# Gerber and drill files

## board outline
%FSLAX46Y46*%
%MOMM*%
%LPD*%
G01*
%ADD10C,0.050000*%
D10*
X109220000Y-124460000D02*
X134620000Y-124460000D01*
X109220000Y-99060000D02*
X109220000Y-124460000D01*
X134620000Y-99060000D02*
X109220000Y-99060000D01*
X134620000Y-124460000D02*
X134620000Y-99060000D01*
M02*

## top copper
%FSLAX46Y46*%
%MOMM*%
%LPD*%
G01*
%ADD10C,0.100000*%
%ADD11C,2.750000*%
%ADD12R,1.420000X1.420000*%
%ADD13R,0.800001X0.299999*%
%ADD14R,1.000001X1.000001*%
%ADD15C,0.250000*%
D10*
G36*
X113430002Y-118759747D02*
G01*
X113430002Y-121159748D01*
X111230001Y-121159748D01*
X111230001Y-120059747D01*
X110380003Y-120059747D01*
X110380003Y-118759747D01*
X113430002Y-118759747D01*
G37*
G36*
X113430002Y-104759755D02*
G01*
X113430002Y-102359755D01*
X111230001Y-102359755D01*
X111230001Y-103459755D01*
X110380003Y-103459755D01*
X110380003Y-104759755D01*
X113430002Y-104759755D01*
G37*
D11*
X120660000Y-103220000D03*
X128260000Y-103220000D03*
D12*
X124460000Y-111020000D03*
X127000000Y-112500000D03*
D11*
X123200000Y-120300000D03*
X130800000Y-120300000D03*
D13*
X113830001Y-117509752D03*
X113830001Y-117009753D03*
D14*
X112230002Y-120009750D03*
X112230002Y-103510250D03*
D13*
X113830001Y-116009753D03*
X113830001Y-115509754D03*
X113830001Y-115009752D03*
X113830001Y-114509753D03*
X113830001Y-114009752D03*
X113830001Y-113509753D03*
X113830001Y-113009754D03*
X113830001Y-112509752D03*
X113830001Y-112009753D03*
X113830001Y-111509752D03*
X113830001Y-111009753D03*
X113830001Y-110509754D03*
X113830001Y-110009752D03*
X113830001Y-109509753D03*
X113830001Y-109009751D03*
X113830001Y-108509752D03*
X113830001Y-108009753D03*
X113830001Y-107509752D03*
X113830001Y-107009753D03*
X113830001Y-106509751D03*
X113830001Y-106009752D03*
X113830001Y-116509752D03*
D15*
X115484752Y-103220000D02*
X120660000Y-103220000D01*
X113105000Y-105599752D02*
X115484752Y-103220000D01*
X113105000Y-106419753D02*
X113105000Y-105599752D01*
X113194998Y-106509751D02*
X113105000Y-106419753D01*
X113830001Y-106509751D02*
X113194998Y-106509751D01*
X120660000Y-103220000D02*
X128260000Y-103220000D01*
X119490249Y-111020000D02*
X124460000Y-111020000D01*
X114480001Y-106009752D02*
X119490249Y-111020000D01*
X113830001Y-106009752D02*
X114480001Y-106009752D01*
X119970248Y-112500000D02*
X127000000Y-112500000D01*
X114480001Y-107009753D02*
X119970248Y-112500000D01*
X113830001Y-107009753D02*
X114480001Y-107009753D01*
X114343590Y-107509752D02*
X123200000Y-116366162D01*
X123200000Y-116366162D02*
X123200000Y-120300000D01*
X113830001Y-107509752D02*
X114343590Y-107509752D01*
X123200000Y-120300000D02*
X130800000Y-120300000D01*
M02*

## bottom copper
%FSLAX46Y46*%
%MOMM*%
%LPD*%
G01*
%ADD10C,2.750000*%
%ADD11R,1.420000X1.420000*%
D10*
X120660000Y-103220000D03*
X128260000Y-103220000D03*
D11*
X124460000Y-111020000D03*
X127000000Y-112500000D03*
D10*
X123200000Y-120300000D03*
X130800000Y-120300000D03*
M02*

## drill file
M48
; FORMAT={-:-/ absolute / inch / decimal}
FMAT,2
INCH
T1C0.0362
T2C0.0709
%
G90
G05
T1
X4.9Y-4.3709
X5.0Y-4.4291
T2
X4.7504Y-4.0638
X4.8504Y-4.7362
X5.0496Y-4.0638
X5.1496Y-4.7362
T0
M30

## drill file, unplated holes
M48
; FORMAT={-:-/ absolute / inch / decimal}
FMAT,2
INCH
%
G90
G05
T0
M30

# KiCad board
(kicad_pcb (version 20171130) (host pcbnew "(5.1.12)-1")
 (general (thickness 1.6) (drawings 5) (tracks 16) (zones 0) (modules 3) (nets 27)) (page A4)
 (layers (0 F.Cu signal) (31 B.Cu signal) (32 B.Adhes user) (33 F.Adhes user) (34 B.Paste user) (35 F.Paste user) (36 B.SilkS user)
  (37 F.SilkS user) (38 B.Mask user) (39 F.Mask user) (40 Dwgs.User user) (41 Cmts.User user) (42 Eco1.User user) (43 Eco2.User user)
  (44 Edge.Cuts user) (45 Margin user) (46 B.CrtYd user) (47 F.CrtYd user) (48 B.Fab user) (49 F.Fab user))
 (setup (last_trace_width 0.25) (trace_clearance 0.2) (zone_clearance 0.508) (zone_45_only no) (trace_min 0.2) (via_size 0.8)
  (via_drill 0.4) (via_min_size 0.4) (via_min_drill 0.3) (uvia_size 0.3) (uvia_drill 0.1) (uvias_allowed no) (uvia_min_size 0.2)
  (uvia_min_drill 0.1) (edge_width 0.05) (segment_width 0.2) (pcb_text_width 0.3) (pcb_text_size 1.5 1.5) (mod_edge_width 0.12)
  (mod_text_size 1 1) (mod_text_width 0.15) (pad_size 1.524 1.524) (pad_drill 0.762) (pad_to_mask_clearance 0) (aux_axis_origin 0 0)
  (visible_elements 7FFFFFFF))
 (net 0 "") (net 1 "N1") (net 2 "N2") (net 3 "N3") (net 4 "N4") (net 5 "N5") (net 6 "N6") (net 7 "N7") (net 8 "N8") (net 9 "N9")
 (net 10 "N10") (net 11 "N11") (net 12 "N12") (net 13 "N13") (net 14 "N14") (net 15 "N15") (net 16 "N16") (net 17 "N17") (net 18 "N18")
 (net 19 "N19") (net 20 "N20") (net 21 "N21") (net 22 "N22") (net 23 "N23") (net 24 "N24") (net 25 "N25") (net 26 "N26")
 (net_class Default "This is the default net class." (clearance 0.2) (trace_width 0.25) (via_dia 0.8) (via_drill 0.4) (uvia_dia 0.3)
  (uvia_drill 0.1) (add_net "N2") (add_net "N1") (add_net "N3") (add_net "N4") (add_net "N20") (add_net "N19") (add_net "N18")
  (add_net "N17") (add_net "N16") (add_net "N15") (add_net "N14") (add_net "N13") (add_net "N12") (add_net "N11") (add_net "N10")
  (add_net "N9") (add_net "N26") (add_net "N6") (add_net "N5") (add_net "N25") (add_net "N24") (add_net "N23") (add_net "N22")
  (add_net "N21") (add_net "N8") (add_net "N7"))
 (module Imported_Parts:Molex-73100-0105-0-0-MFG (layer F.Cu) (at 124.46 96.52 180)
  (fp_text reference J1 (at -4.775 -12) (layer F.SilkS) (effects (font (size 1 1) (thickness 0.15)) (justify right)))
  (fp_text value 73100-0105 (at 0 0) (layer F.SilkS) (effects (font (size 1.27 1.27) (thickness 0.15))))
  (pad 3 thru_hole circle (at 3.8 -6.7 180) (size 2.75 2.75) (drill 1.8) (layers *.Cu) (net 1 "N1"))
  (pad 2 thru_hole circle (at -3.8 -6.7 180) (size 2.75 2.75) (drill 1.8) (layers *.Cu) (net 1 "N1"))
  (pad 1 thru_hole rect (at 0 -14.5 180) (size 1.42 1.42) (drill 0.92) (layers *.Cu) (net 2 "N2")))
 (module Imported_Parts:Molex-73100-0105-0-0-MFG (layer F.Cu) (at 127 127)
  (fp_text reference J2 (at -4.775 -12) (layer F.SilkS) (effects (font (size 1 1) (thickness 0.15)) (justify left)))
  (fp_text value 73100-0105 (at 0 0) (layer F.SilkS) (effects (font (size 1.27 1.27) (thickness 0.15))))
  (pad 1 thru_hole rect (at 0 -14.5) (size 1.42 1.42) (drill 0.92) (layers *.Cu) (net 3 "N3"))
  (pad 2 thru_hole circle (at -3.8 -6.7) (size 2.75 2.75) (drill 1.8) (layers *.Cu) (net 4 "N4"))
  (pad 3 thru_hole circle (at 3.8 -6.7) (size 2.75 2.75) (drill 1.8) (layers *.Cu) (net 4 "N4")))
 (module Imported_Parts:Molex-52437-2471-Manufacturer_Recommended (layer F.Cu) (at 113.03 111.76 270)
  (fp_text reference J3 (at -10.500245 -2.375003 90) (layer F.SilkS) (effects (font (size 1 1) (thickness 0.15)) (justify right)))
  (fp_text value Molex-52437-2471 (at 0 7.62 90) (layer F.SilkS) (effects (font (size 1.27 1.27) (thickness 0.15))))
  (fp_poly
   (pts (xy 6.999747 -0.400002) (xy 9.399748 -0.400002) (xy 9.399748 1.799999) (xy 8.299747 1.799999) (xy 8.299747 2.649997)
    (xy 6.999747 2.649997))
   (layer F.Cu) (width 0))
  (fp_poly
   (pts (xy -7.000245 -0.400002) (xy -9.400245 -0.400002) (xy -9.400245 1.799999) (xy -8.300245 1.799999) (xy -8.300245 2.649997)
    (xy -7.000245 2.649997))
   (layer F.Cu) (width 0))
  (pad 24 smd rect (at 5.749752 -0.800001 270) (size 0.299999 0.800001) (layers F.Cu F.Paste F.Mask) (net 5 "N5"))
  (pad 23 smd rect (at 5.249753 -0.800001 270) (size 0.299999 0.800001) (layers F.Cu F.Paste F.Mask) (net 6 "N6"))
  (pad MP2 smd rect (at 8.24975 0.799998 90) (size 1.000001 1.000001) (layers F.Cu F.Paste F.Mask) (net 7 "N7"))
  (pad MP1 smd rect (at -8.24975 0.799998 90) (size 1.000001 1.000001) (layers F.Cu F.Paste F.Mask) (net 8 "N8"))
  (pad 21 smd rect (at 4.249753 -0.800001 90) (size 0.299999 0.800001) (layers F.Cu F.Paste F.Mask) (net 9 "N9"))
  (pad 20 smd rect (at 3.749754 -0.800001 90) (size 0.299999 0.800001) (layers F.Cu F.Paste F.Mask) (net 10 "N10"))
  (pad 19 smd rect (at 3.249752 -0.800001 90) (size 0.299999 0.800001) (layers F.Cu F.Paste F.Mask) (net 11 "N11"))
  (pad 18 smd rect (at 2.749753 -0.800001 90) (size 0.299999 0.800001) (layers F.Cu F.Paste F.Mask) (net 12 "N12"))
  (pad 17 smd rect (at 2.249752 -0.800001 90) (size 0.299999 0.800001) (layers F.Cu F.Paste F.Mask) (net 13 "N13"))
  (pad 16 smd rect (at 1.749753 -0.800001 90) (size 0.299999 0.800001) (layers F.Cu F.Paste F.Mask) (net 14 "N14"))
  (pad 15 smd rect (at 1.249754 -0.800001 90) (size 0.299999 0.800001) (layers F.Cu F.Paste F.Mask) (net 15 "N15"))
  (pad 14 smd rect (at 0.749752 -0.800001 90) (size 0.299999 0.800001) (layers F.Cu F.Paste F.Mask) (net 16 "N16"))
  (pad 13 smd rect (at 0.249753 -0.800001 90) (size 0.299999 0.800001) (layers F.Cu F.Paste F.Mask) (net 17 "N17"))
  (pad 12 smd rect (at -0.250248 -0.800001 90) (size 0.299999 0.800001) (layers F.Cu F.Paste F.Mask) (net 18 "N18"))
  (pad 11 smd rect (at -0.750247 -0.800001 90) (size 0.299999 0.800001) (layers F.Cu F.Paste F.Mask) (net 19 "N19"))
  (pad 10 smd rect (at -1.250246 -0.800001 90) (size 0.299999 0.800001) (layers F.Cu F.Paste F.Mask) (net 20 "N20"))
  (pad 9 smd rect (at -1.750248 -0.800001 90) (size 0.299999 0.800001) (layers F.Cu F.Paste F.Mask) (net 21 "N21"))
  (pad 8 smd rect (at -2.250247 -0.800001 90) (size 0.299999 0.800001) (layers F.Cu F.Paste F.Mask) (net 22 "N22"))
  (pad 7 smd rect (at -2.750249 -0.800001 90) (size 0.299999 0.800001) (layers F.Cu F.Paste F.Mask) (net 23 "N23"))
  (pad 6 smd rect (at -3.250248 -0.800001 90) (size 0.299999 0.800001) (layers F.Cu F.Paste F.Mask) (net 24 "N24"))
  (pad 5 smd rect (at -3.750247 -0.800001 90) (size 0.299999 0.800001) (layers F.Cu F.Paste F.Mask) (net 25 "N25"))
  (pad 4 smd rect (at -4.250248 -0.800001 90) (size 0.299999 0.800001) (layers F.Cu F.Paste F.Mask) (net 4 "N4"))
  (pad 3 smd rect (at -4.750247 -0.800001 90) (size 0.299999 0.800001) (layers F.Cu F.Paste F.Mask) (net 3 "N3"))
  (pad 2 smd rect (at -5.250249 -0.800001 90) (size 0.299999 0.800001) (layers F.Cu F.Paste F.Mask) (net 1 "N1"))
  (pad 1 smd rect (at -5.750248 -0.800001 90) (size 0.299999 0.800001) (layers F.Cu F.Paste F.Mask) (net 2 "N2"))
  (pad 22 smd rect (at 4.749752 -0.800001 270) (size 0.299999 0.800001) (layers F.Cu F.Paste F.Mask) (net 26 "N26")))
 (gr_line (start 109.22 124.46) (end 134.62 124.46) (layer Edge.Cuts) (width 0.05))
 (gr_line (start 109.22 99.06) (end 109.22 124.46) (layer Edge.Cuts) (width 0.05))
 (gr_line (start 134.62 99.06) (end 109.22 99.06) (layer Edge.Cuts) (width 0.05))
 (gr_line (start 134.62 124.46) (end 134.62 99.06) (layer Edge.Cuts) (width 0.05))
 (segment (start 115.484752 103.22) (end 120.66 103.22) (width 0.25) (layer F.Cu) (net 1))
 (segment (start 113.105 105.599752) (end 115.484752 103.22) (width 0.25) (layer F.Cu) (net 1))
 (segment (start 113.105 106.419753) (end 113.105 105.599752) (width 0.25) (layer F.Cu) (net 1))
 (segment (start 113.194998 106.509751) (end 113.105 106.419753) (width 0.25) (layer F.Cu) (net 1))
 (segment (start 113.830001 106.509751) (end 113.194998 106.509751) (width 0.25) (layer F.Cu) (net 1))
 (segment (start 120.66 103.22) (end 128.26 103.22) (width 0.25) (layer F.Cu) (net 1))
 (segment (start 119.490249 111.02) (end 124.46 111.02) (width 0.25) (layer F.Cu) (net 2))
 (segment (start 114.480001 106.009752) (end 119.490249 111.02) (width 0.25) (layer F.Cu) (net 2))
 (segment (start 113.830001 106.009752) (end 114.480001 106.009752) (width 0.25) (layer F.Cu) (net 2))
 (segment (start 119.970248 112.5) (end 127 112.5) (width 0.25) (layer F.Cu) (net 3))
 (segment (start 114.480001 107.009753) (end 119.970248 112.5) (width 0.25) (layer F.Cu) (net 3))
 (segment (start 113.830001 107.009753) (end 114.480001 107.009753) (width 0.25) (layer F.Cu) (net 3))
 (segment (start 114.34359 107.509752) (end 123.2 116.366162) (width 0.25) (layer F.Cu) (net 4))
 (segment (start 123.2 116.366162) (end 123.2 120.3) (width 0.25) (layer F.Cu) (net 4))
 (segment (start 113.830001 107.509752) (end 114.34359 107.509752) (width 0.25) (layer F.Cu) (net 4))
 (segment (start 123.2 120.3) (end 130.8 120.3) (width 0.25) (layer F.Cu) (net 4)))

